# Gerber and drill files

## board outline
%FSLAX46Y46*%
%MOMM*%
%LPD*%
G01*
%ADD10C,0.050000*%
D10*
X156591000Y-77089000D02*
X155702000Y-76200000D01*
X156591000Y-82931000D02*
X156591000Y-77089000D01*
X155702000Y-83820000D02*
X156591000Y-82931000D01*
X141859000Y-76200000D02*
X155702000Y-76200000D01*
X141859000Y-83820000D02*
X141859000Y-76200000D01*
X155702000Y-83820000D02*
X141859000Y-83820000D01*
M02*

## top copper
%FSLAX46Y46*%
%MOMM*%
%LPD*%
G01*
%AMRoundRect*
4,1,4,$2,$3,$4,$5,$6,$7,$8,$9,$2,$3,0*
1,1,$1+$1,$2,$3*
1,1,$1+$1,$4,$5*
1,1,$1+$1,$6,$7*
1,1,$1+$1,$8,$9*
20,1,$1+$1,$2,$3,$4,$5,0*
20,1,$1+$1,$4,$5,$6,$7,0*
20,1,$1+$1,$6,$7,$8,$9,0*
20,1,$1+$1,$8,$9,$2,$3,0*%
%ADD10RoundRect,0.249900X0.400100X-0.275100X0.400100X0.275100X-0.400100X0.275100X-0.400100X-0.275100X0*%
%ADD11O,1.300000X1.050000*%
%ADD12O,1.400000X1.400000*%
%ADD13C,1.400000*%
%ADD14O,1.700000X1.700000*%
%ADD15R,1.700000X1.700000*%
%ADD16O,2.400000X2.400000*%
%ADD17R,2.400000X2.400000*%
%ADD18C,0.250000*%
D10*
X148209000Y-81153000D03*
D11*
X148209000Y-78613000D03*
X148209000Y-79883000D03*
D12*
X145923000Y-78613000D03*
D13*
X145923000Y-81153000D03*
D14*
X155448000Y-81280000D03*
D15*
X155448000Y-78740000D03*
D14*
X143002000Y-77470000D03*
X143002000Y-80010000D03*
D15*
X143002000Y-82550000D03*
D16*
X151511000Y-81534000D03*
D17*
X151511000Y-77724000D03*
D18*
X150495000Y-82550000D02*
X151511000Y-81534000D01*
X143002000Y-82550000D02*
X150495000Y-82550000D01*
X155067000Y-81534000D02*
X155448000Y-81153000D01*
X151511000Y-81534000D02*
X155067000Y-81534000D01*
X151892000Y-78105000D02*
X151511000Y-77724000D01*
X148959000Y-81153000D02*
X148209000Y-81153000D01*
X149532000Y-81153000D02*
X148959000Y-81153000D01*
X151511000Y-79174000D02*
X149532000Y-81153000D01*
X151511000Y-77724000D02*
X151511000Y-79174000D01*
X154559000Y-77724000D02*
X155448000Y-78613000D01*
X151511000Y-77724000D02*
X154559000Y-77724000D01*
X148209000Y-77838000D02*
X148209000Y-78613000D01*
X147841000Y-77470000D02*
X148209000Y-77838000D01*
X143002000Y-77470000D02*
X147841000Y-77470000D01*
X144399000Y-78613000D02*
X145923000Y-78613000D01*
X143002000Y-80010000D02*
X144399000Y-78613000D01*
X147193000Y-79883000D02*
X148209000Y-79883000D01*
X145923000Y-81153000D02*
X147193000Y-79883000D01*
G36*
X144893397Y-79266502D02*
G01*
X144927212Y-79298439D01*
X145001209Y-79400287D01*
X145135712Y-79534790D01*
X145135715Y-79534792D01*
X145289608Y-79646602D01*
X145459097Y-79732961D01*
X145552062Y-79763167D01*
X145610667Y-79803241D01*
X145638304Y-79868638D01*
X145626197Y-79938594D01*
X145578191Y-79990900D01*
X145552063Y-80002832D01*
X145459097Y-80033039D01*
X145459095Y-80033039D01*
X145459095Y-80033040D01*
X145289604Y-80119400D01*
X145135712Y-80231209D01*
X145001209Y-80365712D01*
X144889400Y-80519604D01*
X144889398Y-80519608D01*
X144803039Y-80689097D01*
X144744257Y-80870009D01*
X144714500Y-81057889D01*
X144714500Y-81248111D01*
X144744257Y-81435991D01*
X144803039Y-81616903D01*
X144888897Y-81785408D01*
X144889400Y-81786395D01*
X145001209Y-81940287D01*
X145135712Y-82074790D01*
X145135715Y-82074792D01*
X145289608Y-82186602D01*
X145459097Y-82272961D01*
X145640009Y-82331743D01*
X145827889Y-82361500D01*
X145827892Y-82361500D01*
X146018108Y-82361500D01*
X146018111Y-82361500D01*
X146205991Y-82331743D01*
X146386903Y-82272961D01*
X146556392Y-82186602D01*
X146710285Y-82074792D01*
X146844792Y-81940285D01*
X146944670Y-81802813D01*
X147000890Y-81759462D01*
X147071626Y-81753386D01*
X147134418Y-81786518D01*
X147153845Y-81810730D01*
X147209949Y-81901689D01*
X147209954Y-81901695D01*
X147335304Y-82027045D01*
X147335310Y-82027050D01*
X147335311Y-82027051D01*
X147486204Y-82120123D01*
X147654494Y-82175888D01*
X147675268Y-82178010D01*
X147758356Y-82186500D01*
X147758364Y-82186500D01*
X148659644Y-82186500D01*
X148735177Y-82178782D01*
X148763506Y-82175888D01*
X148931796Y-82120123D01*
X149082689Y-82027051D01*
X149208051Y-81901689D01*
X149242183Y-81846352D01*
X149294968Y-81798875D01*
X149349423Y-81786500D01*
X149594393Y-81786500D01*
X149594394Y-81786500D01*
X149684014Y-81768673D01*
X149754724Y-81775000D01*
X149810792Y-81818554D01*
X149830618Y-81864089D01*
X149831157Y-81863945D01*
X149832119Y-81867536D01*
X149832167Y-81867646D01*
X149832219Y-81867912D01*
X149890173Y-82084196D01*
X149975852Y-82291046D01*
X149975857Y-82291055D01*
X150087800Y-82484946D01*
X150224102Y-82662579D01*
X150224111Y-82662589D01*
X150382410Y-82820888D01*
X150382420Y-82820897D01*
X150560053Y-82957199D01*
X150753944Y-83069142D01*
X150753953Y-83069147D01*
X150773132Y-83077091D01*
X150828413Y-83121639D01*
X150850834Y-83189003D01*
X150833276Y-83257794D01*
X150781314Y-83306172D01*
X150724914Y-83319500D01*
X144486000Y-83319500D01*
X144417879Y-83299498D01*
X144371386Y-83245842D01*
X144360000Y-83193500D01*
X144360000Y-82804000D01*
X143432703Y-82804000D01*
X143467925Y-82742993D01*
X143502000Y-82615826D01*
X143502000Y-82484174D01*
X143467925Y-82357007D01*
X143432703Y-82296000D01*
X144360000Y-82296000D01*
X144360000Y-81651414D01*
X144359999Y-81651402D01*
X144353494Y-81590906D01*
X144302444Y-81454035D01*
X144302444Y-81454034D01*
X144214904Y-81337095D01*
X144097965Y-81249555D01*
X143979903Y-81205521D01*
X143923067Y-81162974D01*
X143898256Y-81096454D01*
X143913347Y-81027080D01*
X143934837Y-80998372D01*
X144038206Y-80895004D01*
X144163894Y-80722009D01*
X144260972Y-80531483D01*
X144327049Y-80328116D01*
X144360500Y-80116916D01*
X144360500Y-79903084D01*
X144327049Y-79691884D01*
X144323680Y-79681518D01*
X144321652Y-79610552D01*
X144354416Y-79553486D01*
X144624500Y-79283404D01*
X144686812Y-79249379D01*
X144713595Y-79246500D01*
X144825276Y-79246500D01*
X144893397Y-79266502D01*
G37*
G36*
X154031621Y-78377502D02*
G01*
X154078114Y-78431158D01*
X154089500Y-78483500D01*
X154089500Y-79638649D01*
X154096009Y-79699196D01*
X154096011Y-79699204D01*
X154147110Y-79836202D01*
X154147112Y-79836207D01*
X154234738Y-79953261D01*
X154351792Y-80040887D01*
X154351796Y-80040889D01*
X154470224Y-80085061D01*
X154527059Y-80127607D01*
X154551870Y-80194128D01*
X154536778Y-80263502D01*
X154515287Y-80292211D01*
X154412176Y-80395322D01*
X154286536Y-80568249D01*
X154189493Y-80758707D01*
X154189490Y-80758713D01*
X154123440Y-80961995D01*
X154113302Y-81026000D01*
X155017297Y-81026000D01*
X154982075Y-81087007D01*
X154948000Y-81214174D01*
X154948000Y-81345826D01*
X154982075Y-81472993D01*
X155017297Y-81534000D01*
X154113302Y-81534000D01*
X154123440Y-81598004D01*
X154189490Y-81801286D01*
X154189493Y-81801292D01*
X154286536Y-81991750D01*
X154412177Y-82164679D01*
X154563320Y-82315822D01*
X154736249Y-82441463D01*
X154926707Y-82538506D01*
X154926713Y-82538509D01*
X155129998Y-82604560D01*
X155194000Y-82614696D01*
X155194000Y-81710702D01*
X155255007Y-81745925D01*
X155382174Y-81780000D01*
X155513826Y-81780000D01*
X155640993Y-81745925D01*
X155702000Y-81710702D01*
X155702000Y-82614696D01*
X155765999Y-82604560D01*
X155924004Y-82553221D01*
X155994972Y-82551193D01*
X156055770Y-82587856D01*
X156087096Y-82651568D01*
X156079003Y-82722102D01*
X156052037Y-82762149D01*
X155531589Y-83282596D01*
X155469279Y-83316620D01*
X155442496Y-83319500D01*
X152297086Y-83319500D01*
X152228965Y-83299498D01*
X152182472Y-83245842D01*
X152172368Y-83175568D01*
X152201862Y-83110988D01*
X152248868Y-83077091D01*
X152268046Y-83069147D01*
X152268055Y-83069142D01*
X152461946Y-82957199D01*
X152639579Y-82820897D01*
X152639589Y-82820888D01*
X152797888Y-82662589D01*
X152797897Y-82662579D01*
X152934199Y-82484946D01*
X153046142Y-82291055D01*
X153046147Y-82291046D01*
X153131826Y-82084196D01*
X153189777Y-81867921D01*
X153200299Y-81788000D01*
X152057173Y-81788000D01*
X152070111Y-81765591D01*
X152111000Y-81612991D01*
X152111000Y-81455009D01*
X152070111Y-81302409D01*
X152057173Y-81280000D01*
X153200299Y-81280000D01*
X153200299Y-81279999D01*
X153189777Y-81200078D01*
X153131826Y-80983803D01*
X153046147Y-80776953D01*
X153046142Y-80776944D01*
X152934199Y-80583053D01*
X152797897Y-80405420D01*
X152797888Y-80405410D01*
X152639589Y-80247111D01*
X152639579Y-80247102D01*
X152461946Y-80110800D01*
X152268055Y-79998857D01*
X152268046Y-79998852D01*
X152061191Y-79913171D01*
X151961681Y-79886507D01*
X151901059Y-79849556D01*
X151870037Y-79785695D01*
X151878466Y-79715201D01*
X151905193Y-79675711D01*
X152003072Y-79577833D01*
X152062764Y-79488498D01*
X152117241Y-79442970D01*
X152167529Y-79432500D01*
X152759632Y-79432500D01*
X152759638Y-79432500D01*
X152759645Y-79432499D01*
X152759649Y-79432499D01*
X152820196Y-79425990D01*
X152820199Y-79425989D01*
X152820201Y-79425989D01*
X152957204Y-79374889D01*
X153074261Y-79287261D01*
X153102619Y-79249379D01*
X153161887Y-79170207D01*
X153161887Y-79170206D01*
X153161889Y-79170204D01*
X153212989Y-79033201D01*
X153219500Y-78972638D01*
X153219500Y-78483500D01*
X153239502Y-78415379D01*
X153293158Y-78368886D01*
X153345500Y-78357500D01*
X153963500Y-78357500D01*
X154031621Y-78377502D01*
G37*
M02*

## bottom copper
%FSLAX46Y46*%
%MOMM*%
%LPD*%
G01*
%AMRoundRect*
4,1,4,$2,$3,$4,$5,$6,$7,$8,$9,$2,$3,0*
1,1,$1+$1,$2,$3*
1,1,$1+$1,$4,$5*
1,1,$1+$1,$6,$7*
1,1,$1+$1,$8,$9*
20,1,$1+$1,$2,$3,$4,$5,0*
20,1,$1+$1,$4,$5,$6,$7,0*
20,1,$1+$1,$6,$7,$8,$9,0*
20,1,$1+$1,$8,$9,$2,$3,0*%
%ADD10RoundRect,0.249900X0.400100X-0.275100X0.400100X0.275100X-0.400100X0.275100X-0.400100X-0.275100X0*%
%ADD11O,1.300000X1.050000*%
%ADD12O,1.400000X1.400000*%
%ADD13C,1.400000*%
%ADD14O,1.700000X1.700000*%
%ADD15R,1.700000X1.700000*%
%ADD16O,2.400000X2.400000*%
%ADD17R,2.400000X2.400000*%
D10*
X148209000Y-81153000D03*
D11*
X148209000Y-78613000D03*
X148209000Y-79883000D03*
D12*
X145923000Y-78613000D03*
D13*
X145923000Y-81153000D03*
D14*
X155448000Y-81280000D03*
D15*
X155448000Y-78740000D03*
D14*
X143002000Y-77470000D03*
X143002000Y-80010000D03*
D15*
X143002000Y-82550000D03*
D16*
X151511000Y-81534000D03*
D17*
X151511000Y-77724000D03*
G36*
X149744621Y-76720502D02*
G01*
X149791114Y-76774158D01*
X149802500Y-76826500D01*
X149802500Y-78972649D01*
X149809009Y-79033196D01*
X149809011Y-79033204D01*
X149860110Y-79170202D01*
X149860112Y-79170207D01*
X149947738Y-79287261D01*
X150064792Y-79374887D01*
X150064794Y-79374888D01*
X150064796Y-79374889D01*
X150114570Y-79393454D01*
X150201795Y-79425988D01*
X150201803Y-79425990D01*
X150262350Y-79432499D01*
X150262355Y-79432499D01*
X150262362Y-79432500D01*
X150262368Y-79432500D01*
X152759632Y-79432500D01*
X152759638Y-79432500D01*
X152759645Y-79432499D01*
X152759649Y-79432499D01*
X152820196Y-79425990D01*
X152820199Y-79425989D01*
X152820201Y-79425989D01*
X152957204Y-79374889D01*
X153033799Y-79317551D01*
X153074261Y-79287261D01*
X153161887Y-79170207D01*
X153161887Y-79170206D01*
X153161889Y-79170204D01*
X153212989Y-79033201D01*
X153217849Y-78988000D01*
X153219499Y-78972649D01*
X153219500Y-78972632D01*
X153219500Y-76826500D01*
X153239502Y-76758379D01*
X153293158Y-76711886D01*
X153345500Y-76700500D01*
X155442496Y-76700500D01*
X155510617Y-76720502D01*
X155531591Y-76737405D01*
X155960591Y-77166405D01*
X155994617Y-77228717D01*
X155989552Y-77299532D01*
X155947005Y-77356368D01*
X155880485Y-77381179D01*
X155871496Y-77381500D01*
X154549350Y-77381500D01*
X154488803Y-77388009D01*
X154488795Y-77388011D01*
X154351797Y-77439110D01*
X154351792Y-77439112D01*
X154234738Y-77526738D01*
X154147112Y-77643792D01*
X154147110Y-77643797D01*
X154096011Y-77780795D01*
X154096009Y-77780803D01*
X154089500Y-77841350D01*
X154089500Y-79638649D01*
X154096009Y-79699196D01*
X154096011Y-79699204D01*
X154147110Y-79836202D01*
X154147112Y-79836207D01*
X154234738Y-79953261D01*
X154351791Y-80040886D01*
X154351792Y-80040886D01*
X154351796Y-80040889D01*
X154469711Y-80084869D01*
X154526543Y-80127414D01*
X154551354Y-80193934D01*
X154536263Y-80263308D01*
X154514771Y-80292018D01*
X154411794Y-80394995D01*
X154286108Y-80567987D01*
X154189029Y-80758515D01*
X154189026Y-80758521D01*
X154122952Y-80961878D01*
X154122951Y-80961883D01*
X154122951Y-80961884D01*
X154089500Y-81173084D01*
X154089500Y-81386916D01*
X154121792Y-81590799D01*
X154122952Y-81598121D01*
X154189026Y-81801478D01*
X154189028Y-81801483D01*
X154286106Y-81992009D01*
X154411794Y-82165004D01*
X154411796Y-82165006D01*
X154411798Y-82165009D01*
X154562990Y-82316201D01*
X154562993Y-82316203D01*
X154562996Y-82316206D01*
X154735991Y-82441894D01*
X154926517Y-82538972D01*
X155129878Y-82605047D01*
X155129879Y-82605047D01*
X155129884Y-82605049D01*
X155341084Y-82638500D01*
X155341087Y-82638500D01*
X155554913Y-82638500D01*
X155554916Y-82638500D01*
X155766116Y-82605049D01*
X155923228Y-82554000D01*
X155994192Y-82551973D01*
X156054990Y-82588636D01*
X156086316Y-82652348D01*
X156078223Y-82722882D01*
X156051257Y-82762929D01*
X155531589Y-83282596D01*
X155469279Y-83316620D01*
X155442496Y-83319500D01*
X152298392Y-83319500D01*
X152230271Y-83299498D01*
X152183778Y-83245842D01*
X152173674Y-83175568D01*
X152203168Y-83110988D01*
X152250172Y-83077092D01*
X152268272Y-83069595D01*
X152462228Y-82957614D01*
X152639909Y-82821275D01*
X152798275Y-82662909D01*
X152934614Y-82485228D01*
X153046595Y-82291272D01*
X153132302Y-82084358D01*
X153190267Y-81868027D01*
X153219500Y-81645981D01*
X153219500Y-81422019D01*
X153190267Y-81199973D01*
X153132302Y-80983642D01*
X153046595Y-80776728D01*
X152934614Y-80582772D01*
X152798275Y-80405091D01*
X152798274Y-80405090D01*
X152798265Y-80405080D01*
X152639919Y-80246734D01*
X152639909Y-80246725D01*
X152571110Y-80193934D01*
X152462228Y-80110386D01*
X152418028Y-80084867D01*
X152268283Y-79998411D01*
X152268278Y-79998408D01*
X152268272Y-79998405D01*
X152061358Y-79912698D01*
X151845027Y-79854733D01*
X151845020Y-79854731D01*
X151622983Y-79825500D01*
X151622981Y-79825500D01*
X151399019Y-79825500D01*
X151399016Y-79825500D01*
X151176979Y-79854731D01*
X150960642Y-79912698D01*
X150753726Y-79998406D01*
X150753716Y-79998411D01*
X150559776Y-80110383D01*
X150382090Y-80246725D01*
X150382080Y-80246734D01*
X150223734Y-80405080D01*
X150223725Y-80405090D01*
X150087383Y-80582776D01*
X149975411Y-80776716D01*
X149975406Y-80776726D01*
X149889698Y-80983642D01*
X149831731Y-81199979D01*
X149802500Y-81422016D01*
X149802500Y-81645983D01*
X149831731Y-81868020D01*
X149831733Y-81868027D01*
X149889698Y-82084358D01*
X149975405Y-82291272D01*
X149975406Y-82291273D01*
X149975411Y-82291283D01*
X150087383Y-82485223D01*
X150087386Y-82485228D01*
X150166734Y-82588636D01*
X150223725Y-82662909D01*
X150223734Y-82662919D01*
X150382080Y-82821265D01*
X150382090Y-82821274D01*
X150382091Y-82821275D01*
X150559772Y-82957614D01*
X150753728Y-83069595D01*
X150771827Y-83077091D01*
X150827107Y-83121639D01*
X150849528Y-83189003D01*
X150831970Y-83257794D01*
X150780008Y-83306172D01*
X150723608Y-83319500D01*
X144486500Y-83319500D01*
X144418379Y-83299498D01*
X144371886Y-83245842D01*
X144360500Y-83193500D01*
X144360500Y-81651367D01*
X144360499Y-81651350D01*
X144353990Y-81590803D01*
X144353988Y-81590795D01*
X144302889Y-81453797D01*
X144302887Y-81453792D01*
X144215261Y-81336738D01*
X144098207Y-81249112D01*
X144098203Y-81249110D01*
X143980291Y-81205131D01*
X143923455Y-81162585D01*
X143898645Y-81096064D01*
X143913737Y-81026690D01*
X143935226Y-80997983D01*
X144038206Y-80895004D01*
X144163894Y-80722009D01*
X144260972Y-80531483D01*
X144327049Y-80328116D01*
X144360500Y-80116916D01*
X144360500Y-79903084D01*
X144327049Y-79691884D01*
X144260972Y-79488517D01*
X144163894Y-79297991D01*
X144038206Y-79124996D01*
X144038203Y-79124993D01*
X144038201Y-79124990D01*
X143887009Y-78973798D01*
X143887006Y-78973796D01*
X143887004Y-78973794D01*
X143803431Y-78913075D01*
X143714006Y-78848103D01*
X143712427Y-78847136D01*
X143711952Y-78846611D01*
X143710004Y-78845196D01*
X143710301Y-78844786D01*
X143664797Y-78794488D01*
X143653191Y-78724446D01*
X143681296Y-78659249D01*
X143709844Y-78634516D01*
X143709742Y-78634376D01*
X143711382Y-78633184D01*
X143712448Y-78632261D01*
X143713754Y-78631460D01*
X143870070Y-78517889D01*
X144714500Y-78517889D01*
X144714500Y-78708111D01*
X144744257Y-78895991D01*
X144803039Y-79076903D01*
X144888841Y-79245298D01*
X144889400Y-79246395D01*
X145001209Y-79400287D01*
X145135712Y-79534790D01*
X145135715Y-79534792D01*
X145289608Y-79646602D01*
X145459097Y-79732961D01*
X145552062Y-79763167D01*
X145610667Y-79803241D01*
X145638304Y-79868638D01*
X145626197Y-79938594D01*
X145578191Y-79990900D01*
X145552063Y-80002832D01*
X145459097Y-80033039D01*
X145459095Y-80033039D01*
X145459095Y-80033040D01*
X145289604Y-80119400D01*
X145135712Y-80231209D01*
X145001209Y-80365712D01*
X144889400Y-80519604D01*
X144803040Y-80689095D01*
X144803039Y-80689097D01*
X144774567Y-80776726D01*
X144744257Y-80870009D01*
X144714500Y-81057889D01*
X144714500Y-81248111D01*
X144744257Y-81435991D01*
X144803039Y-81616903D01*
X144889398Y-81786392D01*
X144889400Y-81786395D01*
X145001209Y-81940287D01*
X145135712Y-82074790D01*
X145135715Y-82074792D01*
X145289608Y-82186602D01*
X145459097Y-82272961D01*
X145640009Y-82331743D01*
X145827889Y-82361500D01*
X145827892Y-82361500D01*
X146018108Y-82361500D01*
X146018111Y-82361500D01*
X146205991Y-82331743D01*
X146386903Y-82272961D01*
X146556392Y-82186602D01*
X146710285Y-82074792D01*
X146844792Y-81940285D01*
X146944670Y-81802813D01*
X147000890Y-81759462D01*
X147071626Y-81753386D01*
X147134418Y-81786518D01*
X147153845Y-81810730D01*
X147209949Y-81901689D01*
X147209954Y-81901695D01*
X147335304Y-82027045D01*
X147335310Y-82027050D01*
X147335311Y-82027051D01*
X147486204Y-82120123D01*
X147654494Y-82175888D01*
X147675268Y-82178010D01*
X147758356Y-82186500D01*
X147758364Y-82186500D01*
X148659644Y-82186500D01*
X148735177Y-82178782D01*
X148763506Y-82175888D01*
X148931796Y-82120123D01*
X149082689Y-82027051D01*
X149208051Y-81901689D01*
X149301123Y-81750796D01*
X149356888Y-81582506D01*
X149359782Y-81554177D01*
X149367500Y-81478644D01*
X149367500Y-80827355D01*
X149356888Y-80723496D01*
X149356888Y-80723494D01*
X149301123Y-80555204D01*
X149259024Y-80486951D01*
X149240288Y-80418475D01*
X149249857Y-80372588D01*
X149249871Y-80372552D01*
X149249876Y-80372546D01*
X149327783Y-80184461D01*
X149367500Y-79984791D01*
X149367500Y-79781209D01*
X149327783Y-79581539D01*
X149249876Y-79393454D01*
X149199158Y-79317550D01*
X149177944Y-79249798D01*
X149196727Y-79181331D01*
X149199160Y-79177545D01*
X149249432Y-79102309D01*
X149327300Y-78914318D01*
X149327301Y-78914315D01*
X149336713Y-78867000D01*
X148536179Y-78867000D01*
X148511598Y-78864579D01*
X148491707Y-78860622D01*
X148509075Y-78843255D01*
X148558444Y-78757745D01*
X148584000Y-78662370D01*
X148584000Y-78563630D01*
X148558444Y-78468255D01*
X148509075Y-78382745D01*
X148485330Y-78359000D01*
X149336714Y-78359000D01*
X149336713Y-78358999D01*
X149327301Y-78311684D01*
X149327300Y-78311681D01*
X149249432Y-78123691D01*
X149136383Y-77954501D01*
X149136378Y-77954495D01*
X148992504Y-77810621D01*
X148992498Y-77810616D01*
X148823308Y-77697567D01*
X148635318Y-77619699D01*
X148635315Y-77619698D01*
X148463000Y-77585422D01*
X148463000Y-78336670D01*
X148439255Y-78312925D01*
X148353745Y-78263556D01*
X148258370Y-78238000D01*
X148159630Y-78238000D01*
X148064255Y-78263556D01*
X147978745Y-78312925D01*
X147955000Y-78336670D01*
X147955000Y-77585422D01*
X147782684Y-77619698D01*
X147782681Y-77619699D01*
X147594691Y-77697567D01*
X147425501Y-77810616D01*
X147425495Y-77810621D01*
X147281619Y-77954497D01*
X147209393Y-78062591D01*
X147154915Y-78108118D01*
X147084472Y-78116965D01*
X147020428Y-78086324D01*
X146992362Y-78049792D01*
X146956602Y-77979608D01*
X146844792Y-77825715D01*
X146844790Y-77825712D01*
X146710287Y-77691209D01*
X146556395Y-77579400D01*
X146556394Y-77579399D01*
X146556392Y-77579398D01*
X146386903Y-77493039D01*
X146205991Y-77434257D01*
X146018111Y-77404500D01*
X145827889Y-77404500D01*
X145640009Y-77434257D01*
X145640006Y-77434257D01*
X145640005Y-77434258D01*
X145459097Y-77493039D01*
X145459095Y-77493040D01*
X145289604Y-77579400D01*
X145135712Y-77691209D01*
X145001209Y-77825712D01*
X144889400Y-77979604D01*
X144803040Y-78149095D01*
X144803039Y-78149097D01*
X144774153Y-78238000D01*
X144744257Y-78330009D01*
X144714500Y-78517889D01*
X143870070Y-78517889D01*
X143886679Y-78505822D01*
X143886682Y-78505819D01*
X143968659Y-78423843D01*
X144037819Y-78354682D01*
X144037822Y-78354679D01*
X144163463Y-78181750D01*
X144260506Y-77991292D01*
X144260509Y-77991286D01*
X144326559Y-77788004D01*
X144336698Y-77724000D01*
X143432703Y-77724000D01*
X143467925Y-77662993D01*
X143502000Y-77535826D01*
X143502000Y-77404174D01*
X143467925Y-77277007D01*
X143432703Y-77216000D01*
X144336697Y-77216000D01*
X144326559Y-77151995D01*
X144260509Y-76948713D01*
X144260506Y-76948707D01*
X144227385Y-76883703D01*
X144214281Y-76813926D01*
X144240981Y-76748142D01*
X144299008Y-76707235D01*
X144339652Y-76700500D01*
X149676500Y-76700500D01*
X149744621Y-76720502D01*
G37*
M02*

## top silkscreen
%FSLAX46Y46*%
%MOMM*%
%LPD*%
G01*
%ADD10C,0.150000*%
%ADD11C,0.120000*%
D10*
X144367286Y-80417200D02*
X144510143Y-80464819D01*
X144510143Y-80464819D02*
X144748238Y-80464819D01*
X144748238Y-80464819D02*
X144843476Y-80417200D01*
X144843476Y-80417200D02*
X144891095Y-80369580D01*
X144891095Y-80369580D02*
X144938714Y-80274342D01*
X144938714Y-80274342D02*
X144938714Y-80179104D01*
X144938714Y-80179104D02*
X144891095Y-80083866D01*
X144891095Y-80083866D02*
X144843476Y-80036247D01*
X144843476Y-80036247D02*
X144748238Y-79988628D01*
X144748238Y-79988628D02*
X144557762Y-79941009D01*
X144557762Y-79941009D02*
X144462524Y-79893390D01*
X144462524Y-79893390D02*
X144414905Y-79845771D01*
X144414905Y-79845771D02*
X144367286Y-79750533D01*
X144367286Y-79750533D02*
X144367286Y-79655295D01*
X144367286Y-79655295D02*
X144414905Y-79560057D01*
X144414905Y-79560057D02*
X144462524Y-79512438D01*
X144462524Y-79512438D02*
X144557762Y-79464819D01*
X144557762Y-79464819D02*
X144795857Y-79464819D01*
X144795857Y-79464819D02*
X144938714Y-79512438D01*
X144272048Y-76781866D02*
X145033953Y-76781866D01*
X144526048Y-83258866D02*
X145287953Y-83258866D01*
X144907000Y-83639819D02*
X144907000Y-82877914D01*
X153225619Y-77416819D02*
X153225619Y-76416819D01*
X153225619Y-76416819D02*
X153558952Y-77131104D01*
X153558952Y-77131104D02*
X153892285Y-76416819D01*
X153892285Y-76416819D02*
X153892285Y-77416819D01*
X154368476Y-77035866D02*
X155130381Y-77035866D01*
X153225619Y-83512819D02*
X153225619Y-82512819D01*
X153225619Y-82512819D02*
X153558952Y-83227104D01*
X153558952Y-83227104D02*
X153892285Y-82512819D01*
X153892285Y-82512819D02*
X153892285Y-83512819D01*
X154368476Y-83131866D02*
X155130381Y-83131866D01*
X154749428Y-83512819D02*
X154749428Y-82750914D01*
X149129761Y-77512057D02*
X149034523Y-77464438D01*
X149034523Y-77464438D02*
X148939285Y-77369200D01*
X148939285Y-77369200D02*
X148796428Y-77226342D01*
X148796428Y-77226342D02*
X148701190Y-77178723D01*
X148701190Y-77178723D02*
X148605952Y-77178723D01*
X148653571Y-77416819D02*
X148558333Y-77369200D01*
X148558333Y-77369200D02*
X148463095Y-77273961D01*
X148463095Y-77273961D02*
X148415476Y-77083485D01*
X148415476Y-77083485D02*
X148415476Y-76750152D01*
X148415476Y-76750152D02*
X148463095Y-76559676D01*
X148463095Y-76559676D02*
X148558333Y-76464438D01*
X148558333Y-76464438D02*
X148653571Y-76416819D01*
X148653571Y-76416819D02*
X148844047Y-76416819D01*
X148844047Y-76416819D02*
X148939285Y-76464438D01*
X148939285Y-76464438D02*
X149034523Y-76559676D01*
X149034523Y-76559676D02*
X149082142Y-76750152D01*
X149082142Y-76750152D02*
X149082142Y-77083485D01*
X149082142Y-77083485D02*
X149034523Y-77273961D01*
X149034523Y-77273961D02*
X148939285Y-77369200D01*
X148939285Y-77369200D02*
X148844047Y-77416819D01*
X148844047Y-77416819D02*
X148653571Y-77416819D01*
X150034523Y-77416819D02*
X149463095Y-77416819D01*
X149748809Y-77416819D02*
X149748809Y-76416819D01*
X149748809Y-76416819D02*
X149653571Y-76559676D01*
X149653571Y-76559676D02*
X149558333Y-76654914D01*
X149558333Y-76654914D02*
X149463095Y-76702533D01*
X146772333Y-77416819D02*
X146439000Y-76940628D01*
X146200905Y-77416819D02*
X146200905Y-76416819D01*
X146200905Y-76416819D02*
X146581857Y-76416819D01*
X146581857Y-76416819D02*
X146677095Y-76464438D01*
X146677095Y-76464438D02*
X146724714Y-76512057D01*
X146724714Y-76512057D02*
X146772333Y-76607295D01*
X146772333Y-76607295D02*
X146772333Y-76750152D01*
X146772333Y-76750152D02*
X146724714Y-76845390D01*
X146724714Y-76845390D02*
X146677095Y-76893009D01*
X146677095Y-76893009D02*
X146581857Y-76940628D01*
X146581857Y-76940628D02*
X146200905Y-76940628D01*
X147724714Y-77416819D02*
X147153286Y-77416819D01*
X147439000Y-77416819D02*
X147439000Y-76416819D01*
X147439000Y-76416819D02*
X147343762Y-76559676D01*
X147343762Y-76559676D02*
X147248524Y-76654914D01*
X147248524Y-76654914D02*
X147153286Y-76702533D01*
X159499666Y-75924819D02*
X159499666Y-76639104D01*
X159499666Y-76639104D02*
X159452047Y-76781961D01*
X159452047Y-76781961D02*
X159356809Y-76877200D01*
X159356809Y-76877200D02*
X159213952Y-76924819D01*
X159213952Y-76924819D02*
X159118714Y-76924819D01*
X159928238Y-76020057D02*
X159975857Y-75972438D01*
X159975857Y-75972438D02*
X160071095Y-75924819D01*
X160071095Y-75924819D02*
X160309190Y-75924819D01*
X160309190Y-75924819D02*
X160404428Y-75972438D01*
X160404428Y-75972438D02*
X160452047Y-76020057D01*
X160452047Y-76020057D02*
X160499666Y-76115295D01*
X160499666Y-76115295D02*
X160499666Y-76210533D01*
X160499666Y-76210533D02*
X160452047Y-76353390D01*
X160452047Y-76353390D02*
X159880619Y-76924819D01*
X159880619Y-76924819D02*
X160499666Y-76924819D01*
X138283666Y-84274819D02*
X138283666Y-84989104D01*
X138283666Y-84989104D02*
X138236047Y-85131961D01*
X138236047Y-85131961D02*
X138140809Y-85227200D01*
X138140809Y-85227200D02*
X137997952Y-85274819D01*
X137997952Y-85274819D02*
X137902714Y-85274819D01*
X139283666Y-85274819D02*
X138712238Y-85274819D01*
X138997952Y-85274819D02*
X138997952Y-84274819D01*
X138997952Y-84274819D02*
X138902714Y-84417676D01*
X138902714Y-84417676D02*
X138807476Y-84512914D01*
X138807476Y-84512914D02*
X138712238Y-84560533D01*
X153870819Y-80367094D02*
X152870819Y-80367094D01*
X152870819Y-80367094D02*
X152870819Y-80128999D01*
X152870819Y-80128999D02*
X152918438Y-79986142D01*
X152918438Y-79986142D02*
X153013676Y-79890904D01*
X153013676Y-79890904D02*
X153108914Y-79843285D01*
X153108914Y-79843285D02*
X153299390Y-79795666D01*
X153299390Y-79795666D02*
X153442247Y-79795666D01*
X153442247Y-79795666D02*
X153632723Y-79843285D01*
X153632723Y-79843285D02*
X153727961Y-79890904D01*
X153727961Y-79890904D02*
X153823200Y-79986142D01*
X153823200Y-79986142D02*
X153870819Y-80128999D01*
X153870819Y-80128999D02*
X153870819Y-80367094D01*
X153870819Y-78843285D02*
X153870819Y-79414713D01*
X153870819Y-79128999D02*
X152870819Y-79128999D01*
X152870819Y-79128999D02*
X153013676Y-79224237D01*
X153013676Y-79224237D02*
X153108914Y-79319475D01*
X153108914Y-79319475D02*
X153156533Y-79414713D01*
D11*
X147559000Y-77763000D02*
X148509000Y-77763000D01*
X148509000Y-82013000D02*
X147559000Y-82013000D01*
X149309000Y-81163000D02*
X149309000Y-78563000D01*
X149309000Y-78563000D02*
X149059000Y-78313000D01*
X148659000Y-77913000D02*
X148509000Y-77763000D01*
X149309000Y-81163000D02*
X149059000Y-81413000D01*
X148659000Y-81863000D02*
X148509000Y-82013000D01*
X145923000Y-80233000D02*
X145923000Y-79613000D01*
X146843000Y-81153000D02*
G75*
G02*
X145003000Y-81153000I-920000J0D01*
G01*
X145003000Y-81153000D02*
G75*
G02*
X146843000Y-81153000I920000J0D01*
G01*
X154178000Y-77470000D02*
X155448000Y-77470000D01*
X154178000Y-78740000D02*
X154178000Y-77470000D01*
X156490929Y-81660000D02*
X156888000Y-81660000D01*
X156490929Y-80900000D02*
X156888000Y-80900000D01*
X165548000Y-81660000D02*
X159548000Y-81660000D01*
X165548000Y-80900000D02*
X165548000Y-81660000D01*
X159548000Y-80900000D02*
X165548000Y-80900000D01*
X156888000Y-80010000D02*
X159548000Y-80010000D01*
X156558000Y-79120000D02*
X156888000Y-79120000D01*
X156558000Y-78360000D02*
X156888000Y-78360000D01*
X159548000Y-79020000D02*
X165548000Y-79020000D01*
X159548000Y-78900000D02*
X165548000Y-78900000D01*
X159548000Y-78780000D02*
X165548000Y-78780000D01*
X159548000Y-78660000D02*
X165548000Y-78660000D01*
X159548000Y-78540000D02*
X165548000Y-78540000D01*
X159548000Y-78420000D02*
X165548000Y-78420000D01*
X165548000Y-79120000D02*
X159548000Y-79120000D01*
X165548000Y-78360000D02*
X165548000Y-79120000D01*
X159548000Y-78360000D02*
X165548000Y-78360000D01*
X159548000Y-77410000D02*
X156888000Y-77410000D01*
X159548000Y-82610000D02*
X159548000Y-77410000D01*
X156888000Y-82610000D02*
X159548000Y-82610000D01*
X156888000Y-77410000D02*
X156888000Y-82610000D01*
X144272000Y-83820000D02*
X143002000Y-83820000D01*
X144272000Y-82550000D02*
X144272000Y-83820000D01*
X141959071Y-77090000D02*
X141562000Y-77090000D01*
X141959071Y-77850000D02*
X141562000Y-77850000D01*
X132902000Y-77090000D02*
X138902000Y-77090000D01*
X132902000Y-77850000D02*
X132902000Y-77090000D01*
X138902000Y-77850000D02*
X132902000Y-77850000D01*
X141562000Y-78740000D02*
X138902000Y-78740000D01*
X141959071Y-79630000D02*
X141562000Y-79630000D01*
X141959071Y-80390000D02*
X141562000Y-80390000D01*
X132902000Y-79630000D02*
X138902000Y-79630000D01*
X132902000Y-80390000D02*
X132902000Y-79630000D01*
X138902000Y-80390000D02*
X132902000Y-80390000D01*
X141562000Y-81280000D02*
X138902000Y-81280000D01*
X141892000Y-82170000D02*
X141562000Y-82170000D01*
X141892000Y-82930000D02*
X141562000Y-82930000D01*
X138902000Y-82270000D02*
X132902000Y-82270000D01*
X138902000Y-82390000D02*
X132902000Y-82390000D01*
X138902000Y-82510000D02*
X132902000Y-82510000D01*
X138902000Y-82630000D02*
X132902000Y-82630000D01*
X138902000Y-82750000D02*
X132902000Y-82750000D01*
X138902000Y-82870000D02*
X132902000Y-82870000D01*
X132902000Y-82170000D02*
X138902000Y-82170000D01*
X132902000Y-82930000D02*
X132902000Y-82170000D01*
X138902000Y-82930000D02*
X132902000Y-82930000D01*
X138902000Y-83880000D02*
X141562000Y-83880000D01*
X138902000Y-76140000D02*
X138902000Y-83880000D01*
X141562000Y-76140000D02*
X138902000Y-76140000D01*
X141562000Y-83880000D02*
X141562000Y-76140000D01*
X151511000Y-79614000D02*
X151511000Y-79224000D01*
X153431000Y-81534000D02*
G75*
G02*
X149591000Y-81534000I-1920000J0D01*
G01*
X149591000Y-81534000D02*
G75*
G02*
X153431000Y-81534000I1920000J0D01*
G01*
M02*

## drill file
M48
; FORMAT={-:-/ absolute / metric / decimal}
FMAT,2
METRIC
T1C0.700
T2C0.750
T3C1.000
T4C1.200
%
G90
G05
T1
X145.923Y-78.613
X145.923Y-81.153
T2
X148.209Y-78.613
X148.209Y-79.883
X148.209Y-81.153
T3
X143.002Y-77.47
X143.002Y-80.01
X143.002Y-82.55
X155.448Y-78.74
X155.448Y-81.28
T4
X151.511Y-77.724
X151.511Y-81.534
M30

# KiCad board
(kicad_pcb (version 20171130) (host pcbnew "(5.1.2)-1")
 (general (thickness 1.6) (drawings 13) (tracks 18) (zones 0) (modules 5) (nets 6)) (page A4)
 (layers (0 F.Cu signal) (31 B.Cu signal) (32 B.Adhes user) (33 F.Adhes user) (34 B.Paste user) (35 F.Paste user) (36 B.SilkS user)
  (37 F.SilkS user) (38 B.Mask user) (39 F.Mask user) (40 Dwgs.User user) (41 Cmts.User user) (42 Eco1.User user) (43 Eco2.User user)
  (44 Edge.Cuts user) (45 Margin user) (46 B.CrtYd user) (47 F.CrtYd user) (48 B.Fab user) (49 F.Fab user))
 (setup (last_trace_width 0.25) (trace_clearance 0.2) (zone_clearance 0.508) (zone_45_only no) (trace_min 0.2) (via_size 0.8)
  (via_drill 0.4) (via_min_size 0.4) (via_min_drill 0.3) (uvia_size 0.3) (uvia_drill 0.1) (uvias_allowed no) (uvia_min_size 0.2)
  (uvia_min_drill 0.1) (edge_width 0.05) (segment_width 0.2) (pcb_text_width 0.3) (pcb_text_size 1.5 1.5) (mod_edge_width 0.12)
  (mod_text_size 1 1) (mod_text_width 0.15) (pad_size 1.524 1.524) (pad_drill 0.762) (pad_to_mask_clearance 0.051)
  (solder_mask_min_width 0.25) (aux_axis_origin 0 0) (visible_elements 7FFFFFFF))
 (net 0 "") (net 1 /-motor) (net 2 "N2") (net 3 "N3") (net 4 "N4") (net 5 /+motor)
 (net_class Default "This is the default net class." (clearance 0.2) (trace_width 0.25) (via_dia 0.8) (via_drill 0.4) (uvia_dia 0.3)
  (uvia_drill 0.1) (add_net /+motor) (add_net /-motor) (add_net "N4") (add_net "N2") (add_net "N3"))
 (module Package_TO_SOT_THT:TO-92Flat (layer F.Cu) (at 148.209 81.153 90)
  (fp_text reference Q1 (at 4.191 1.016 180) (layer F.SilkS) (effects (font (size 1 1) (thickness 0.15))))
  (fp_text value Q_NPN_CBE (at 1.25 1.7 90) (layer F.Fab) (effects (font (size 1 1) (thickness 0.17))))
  (fp_line (start 3.39 -0.65) (end 3.39 0.3) (layer F.SilkS) (width 0.12))
  (fp_line (start -0.86 0.3) (end -0.86 -0.65) (layer F.SilkS) (width 0.12))
  (fp_line (start -0.01 1.1) (end 2.59 1.1) (layer F.SilkS) (width 0.12))
  (fp_line (start 2.59 1.1) (end 2.84 0.85) (layer F.SilkS) (width 0.12))
  (fp_line (start 3.24 0.45) (end 3.39 0.3) (layer F.SilkS) (width 0.12))
  (fp_line (start -0.01 1.1) (end -0.26 0.85) (layer F.SilkS) (width 0.12))
  (fp_line (start -0.71 0.45) (end -0.86 0.3) (layer F.SilkS) (width 0.12))
  (pad 1 thru_hole roundrect (at 0 0 90) (size 1.05 1.3) (drill 0.75) (layers *.Cu *.Mask) (roundrect_rratio 0.238) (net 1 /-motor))
  (pad 3 thru_hole oval (at 2.54 0 90) (size 1.05 1.3) (drill 0.75) (layers *.Cu *.Mask) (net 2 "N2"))
  (pad 2 thru_hole oval (at 1.27 0 90) (size 1.05 1.3) (drill 0.75) (layers *.Cu *.Mask) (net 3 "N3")))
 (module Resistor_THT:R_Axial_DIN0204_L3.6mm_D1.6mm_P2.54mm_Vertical (layer F.Cu) (at 145.923 81.153 90)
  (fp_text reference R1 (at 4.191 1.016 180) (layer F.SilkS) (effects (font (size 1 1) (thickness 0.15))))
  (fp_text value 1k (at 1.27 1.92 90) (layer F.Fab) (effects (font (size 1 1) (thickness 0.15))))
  (fp_line (start 0.92 0) (end 1.54 0) (layer F.SilkS) (width 0.12))
  (fp_circle (center 0 0) (end 0.92 0) (layer F.SilkS) (width 0.12))
  (pad 2 thru_hole oval (at 2.54 0 90) (size 1.4 1.4) (drill 0.7) (layers *.Cu *.Mask) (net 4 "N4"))
  (pad 1 thru_hole circle (at 0 0 90) (size 1.4 1.4) (drill 0.7) (layers *.Cu *.Mask) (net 3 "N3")))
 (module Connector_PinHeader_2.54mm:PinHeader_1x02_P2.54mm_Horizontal (layer F.Cu) (at 155.448 78.74)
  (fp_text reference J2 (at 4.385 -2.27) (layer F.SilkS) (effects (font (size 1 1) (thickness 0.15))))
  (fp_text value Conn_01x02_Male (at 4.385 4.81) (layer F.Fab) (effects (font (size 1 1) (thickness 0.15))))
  (fp_line (start -1.27 -1.27) (end 0 -1.27) (layer F.SilkS) (width 0.12))
  (fp_line (start -1.27 0) (end -1.27 -1.27) (layer F.SilkS) (width 0.12))
  (fp_line (start 1.042929 2.92) (end 1.44 2.92) (layer F.SilkS) (width 0.12))
  (fp_line (start 1.042929 2.16) (end 1.44 2.16) (layer F.SilkS) (width 0.12))
  (fp_line (start 10.1 2.92) (end 4.1 2.92) (layer F.SilkS) (width 0.12))
  (fp_line (start 10.1 2.16) (end 10.1 2.92) (layer F.SilkS) (width 0.12))
  (fp_line (start 4.1 2.16) (end 10.1 2.16) (layer F.SilkS) (width 0.12))
  (fp_line (start 1.44 1.27) (end 4.1 1.27) (layer F.SilkS) (width 0.12))
  (fp_line (start 1.11 0.38) (end 1.44 0.38) (layer F.SilkS) (width 0.12))
  (fp_line (start 1.11 -0.38) (end 1.44 -0.38) (layer F.SilkS) (width 0.12))
  (fp_line (start 4.1 0.28) (end 10.1 0.28) (layer F.SilkS) (width 0.12))
  (fp_line (start 4.1 0.16) (end 10.1 0.16) (layer F.SilkS) (width 0.12))
  (fp_line (start 4.1 0.04) (end 10.1 0.04) (layer F.SilkS) (width 0.12))
  (fp_line (start 4.1 -0.08) (end 10.1 -0.08) (layer F.SilkS) (width 0.12))
  (fp_line (start 4.1 -0.2) (end 10.1 -0.2) (layer F.SilkS) (width 0.12))
  (fp_line (start 4.1 -0.32) (end 10.1 -0.32) (layer F.SilkS) (width 0.12))
  (fp_line (start 10.1 0.38) (end 4.1 0.38) (layer F.SilkS) (width 0.12))
  (fp_line (start 10.1 -0.38) (end 10.1 0.38) (layer F.SilkS) (width 0.12))
  (fp_line (start 4.1 -0.38) (end 10.1 -0.38) (layer F.SilkS) (width 0.12))
  (fp_line (start 4.1 -1.33) (end 1.44 -1.33) (layer F.SilkS) (width 0.12))
  (fp_line (start 4.1 3.87) (end 4.1 -1.33) (layer F.SilkS) (width 0.12))
  (fp_line (start 1.44 3.87) (end 4.1 3.87) (layer F.SilkS) (width 0.12))
  (fp_line (start 1.44 -1.33) (end 1.44 3.87) (layer F.SilkS) (width 0.12))
  (pad 2 thru_hole oval (at 0 2.54) (size 1.7 1.7) (drill 1) (layers *.Cu *.Mask) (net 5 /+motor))
  (pad 1 thru_hole rect (at 0 0) (size 1.7 1.7) (drill 1) (layers *.Cu *.Mask) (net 1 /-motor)))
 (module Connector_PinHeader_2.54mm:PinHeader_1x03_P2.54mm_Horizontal (layer F.Cu) (at 143.002 82.55 180)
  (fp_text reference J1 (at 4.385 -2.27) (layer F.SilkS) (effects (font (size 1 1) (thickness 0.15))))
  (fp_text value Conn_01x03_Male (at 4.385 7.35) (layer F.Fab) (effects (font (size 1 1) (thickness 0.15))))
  (fp_line (start -1.27 -1.27) (end 0 -1.27) (layer F.SilkS) (width 0.12))
  (fp_line (start -1.27 0) (end -1.27 -1.27) (layer F.SilkS) (width 0.12))
  (fp_line (start 1.042929 5.46) (end 1.44 5.46) (layer F.SilkS) (width 0.12))
  (fp_line (start 1.042929 4.7) (end 1.44 4.7) (layer F.SilkS) (width 0.12))
  (fp_line (start 10.1 5.46) (end 4.1 5.46) (layer F.SilkS) (width 0.12))
  (fp_line (start 10.1 4.7) (end 10.1 5.46) (layer F.SilkS) (width 0.12))
  (fp_line (start 4.1 4.7) (end 10.1 4.7) (layer F.SilkS) (width 0.12))
  (fp_line (start 1.44 3.81) (end 4.1 3.81) (layer F.SilkS) (width 0.12))
  (fp_line (start 1.042929 2.92) (end 1.44 2.92) (layer F.SilkS) (width 0.12))
  (fp_line (start 1.042929 2.16) (end 1.44 2.16) (layer F.SilkS) (width 0.12))
  (fp_line (start 10.1 2.92) (end 4.1 2.92) (layer F.SilkS) (width 0.12))
  (fp_line (start 10.1 2.16) (end 10.1 2.92) (layer F.SilkS) (width 0.12))
  (fp_line (start 4.1 2.16) (end 10.1 2.16) (layer F.SilkS) (width 0.12))
  (fp_line (start 1.44 1.27) (end 4.1 1.27) (layer F.SilkS) (width 0.12))
  (fp_line (start 1.11 0.38) (end 1.44 0.38) (layer F.SilkS) (width 0.12))
  (fp_line (start 1.11 -0.38) (end 1.44 -0.38) (layer F.SilkS) (width 0.12))
  (fp_line (start 4.1 0.28) (end 10.1 0.28) (layer F.SilkS) (width 0.12))
  (fp_line (start 4.1 0.16) (end 10.1 0.16) (layer F.SilkS) (width 0.12))
  (fp_line (start 4.1 0.04) (end 10.1 0.04) (layer F.SilkS) (width 0.12))
  (fp_line (start 4.1 -0.08) (end 10.1 -0.08) (layer F.SilkS) (width 0.12))
  (fp_line (start 4.1 -0.2) (end 10.1 -0.2) (layer F.SilkS) (width 0.12))
  (fp_line (start 4.1 -0.32) (end 10.1 -0.32) (layer F.SilkS) (width 0.12))
  (fp_line (start 10.1 0.38) (end 4.1 0.38) (layer F.SilkS) (width 0.12))
  (fp_line (start 10.1 -0.38) (end 10.1 0.38) (layer F.SilkS) (width 0.12))
  (fp_line (start 4.1 -0.38) (end 10.1 -0.38) (layer F.SilkS) (width 0.12))
  (fp_line (start 4.1 -1.33) (end 1.44 -1.33) (layer F.SilkS) (width 0.12))
  (fp_line (start 4.1 6.41) (end 4.1 -1.33) (layer F.SilkS) (width 0.12))
  (fp_line (start 1.44 6.41) (end 4.1 6.41) (layer F.SilkS) (width 0.12))
  (fp_line (start 1.44 -1.33) (end 1.44 6.41) (layer F.SilkS) (width 0.12))
  (pad 3 thru_hole oval (at 0 5.08 180) (size 1.7 1.7) (drill 1) (layers *.Cu *.Mask) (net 2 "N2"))
  (pad 2 thru_hole oval (at 0 2.54 180) (size 1.7 1.7) (drill 1) (layers *.Cu *.Mask) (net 4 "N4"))
  (pad 1 thru_hole rect (at 0 0 180) (size 1.7 1.7) (drill 1) (layers *.Cu *.Mask) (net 5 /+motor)))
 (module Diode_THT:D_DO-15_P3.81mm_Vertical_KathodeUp (layer F.Cu) (at 151.511 77.724 270)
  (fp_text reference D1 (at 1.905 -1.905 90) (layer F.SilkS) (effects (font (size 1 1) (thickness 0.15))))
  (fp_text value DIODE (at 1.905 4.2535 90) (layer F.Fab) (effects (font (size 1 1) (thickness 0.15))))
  (fp_line (start 1.89 0) (end 1.5 0) (layer F.SilkS) (width 0.12))
  (fp_circle (center 3.81 0) (end 5.73 0) (layer F.SilkS) (width 0.12))
  (pad 2 thru_hole oval (at 3.81 0 270) (size 2.4 2.4) (drill 1.2) (layers *.Cu *.Mask) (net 5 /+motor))
  (pad 1 thru_hole rect (at 0 0 270) (size 2.4 2.4) (drill 1.2) (layers *.Cu *.Mask) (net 1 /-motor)))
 (gr_line (start 156.591 77.089) (end 155.702 76.2) (layer Edge.Cuts) (width 0.05))
 (gr_line (start 156.591 82.931) (end 156.591 77.089) (layer Edge.Cuts) (width 0.05))
 (gr_line (start 155.702 83.82) (end 156.591 82.931) (layer Edge.Cuts) (width 0.05))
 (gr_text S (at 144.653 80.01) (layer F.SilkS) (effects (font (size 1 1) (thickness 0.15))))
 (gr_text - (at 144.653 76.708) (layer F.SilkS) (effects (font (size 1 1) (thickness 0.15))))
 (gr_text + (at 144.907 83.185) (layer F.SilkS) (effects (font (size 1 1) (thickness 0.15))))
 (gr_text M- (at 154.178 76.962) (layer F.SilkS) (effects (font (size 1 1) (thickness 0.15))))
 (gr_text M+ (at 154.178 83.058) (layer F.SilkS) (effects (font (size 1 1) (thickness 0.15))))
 (gr_line (start 141.859 76.2) (end 155.702 76.2) (layer Edge.Cuts) (width 0.05))
 (gr_line (start 141.859 83.82) (end 141.859 76.2) (layer Edge.Cuts) (width 0.05))
 (gr_line (start 155.702 83.82) (end 141.859 83.82) (layer Edge.Cuts) (width 0.05))
 (segment (start 150.495 82.55) (end 151.511 81.534) (width 0.25) (layer F.Cu) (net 5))
 (segment (start 143.002 82.55) (end 150.495 82.55) (width 0.25) (layer F.Cu) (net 5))
 (segment (start 155.067 81.534) (end 155.448 81.153) (width 0.25) (layer F.Cu) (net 5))
 (segment (start 151.511 81.534) (end 155.067 81.534) (width 0.25) (layer F.Cu) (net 5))
 (segment (start 151.892 78.105) (end 151.511 77.724) (width 0.25) (layer F.Cu) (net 1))
 (segment (start 148.959 81.153) (end 148.209 81.153) (width 0.25) (layer F.Cu) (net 1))
 (segment (start 149.532 81.153) (end 148.959 81.153) (width 0.25) (layer F.Cu) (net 1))
 (segment (start 151.511 79.174) (end 149.532 81.153) (width 0.25) (layer F.Cu) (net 1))
 (segment (start 151.511 77.724) (end 151.511 79.174) (width 0.25) (layer F.Cu) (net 1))
 (segment (start 154.559 77.724) (end 155.448 78.613) (width 0.25) (layer F.Cu) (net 1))
 (segment (start 151.511 77.724) (end 154.559 77.724) (width 0.25) (layer F.Cu) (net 1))
 (segment (start 148.209 77.838) (end 148.209 78.613) (width 0.25) (layer F.Cu) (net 2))
 (segment (start 147.841 77.47) (end 148.209 77.838) (width 0.25) (layer F.Cu) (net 2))
 (segment (start 143.002 77.47) (end 147.841 77.47) (width 0.25) (layer F.Cu) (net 2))
 (segment (start 144.399 78.613) (end 145.923 78.613) (width 0.25) (layer F.Cu) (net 4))
 (segment (start 143.002 80.01) (end 144.399 78.613) (width 0.25) (layer F.Cu) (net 4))
 (segment (start 147.193 79.883) (end 148.209 79.883) (width 0.25) (layer F.Cu) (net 3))
 (segment (start 145.923 81.153) (end 147.193 79.883) (width 0.25) (layer F.Cu) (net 3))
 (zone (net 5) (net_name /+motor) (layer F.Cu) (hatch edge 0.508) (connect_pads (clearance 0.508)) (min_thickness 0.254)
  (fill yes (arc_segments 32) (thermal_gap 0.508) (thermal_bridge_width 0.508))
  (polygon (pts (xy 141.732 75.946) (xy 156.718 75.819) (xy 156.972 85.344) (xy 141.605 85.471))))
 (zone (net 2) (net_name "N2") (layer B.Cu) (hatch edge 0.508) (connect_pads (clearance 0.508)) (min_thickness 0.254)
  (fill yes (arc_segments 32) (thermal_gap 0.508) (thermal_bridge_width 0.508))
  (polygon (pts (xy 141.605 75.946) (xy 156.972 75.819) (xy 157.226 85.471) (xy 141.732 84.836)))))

